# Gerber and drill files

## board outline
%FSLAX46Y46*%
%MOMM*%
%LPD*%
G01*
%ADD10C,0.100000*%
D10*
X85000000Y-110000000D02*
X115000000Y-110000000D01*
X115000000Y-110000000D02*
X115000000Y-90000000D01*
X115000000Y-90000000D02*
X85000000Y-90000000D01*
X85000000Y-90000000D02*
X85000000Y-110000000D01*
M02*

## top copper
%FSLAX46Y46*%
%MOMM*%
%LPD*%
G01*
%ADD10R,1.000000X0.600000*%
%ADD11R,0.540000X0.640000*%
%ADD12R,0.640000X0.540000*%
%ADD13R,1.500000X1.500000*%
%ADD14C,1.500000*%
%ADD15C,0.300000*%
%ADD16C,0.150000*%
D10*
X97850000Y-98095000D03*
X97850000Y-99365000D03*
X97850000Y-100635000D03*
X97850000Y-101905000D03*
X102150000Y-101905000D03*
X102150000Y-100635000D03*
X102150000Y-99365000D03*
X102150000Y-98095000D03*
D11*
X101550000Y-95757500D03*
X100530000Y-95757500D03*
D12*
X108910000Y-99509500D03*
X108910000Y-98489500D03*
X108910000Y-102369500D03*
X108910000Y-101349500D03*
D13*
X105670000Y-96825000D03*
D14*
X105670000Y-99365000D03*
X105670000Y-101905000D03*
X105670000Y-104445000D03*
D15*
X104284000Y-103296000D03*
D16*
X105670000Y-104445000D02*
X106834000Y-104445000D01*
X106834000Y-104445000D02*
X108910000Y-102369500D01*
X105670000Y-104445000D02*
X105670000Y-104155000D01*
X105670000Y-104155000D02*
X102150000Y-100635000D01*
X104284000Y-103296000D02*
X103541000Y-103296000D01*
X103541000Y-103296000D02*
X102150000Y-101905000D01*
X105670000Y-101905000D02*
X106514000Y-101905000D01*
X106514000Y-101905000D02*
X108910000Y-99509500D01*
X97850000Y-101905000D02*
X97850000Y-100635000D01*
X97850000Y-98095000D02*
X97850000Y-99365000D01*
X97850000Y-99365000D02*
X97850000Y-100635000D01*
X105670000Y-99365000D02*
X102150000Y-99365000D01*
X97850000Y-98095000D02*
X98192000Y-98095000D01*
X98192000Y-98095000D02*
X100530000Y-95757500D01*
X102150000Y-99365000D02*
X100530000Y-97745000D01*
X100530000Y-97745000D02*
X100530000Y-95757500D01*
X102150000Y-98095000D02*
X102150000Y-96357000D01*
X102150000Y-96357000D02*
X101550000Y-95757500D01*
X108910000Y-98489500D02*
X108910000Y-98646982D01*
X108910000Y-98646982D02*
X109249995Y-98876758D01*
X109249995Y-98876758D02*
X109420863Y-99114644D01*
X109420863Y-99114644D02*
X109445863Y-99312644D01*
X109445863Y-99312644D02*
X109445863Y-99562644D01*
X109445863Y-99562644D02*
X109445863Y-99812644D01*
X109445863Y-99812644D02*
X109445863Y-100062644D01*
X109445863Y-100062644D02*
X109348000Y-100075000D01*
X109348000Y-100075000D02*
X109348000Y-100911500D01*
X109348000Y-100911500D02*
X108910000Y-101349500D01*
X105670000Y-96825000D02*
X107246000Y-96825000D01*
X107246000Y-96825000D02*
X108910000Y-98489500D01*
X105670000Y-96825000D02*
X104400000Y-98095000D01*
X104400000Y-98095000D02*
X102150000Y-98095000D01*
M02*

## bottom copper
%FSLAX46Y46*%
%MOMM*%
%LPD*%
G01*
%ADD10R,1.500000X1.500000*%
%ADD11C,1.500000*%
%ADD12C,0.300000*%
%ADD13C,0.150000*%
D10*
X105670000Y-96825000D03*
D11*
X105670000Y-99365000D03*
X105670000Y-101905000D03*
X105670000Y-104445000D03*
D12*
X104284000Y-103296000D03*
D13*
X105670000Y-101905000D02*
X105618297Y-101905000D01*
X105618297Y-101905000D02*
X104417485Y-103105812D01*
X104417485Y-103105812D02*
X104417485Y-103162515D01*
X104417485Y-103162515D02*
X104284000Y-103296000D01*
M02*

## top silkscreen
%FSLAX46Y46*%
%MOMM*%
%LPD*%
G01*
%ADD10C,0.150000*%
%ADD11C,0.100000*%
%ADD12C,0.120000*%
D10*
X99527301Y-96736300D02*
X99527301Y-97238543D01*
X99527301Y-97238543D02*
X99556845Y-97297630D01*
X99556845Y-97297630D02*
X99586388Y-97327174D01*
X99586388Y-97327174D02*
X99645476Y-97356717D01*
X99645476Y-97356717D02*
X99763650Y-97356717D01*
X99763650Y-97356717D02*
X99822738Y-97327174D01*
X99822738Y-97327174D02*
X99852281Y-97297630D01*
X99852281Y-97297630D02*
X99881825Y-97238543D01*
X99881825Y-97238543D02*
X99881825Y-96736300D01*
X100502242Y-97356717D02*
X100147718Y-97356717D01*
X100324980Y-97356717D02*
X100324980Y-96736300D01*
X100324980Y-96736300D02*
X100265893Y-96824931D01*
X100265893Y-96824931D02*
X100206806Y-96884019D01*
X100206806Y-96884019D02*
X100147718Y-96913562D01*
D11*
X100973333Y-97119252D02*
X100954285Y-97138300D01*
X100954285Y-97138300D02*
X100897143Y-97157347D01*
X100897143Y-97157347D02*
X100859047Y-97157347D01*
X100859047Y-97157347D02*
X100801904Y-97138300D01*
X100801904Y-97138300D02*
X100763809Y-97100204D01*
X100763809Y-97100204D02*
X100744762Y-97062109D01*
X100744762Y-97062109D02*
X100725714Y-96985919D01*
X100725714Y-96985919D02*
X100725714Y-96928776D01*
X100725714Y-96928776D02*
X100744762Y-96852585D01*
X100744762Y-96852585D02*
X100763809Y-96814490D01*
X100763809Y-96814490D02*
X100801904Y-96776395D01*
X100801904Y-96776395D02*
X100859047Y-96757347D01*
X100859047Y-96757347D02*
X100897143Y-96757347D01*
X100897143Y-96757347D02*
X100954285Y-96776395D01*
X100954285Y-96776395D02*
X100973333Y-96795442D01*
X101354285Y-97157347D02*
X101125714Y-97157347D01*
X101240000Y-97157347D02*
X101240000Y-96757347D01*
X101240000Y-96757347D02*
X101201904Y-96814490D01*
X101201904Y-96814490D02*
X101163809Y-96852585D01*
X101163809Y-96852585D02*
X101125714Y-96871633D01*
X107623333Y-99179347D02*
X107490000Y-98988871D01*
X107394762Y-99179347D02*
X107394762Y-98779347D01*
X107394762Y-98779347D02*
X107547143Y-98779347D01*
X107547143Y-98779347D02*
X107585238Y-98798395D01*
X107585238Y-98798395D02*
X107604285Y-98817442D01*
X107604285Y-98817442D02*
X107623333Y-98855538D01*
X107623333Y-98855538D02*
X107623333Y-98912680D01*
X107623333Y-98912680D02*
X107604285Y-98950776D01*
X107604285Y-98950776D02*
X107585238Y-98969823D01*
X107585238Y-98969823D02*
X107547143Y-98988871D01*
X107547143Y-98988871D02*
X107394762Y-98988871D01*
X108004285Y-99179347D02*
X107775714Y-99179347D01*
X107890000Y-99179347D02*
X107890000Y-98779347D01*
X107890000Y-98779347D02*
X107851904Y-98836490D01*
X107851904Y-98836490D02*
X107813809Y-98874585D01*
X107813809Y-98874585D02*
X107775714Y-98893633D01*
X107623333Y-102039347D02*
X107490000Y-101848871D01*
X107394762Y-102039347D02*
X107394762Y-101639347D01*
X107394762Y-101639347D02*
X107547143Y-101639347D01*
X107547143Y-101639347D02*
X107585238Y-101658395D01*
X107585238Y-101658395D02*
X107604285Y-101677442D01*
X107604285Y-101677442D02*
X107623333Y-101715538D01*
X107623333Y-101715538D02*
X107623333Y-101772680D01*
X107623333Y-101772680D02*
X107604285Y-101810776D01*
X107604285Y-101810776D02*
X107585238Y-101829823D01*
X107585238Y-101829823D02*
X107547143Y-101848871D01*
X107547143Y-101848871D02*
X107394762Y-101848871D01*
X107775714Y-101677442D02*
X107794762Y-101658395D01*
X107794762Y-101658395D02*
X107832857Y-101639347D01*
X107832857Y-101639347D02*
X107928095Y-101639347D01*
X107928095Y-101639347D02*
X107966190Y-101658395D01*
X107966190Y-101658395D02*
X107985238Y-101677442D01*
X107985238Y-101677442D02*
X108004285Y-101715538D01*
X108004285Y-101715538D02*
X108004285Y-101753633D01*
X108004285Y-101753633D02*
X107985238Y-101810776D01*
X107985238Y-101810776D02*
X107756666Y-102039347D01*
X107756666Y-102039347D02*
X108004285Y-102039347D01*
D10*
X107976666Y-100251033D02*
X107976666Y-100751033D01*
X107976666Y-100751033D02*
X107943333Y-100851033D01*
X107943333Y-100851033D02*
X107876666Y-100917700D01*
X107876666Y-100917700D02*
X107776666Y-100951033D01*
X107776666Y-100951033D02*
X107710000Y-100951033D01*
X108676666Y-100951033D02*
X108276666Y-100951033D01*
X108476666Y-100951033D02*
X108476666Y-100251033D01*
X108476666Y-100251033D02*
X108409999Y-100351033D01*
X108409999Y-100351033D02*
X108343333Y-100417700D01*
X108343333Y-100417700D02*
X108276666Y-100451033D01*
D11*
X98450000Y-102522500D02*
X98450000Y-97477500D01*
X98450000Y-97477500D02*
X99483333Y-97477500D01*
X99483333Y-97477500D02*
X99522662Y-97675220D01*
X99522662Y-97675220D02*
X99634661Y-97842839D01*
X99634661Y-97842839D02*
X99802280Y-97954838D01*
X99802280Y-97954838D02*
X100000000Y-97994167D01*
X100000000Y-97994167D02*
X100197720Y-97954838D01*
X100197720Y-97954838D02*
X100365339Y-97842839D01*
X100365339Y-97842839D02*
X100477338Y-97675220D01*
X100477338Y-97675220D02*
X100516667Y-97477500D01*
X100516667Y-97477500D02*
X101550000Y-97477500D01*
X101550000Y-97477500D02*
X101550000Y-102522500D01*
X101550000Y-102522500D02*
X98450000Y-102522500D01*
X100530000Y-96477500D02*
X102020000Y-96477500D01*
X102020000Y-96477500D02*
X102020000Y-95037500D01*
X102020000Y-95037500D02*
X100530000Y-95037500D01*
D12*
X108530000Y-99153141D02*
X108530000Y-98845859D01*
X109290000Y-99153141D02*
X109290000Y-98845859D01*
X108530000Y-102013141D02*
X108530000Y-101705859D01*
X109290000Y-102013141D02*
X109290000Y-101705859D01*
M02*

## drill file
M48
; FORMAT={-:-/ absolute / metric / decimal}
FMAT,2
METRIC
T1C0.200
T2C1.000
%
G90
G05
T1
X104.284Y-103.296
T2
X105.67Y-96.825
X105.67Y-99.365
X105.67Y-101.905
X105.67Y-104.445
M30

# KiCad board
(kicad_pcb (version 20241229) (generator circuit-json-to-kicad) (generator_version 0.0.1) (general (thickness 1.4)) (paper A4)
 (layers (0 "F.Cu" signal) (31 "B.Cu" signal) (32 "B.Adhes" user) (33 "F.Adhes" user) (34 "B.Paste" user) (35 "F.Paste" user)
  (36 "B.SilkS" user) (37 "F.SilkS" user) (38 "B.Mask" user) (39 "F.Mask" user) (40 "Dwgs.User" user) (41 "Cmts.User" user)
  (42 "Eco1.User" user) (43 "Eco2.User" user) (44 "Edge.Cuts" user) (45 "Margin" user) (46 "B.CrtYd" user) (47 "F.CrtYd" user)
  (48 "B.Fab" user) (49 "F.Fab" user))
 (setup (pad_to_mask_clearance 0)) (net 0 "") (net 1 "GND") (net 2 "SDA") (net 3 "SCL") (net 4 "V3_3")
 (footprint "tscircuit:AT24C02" (layer F.Cu) (at 100 100 0)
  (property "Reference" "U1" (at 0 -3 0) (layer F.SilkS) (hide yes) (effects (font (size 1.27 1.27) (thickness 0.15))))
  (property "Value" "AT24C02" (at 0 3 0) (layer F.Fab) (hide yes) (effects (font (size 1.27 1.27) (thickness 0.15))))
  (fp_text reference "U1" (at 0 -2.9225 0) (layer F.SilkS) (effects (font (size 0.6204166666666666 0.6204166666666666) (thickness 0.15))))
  (fp_line (start -1.5499999999999998 2.5225) (end -1.5499999999999998 -2.5225) (stroke (width 0.1) (type default)) (layer F.SilkS))
  (fp_line (start -1.5499999999999998 -2.5225) (end -0.5166666666666666 -2.5225) (stroke (width 0.1) (type default)) (layer F.SilkS))
  (fp_line (start -0.5166666666666666 -2.5225) (end -0.47733775846416476 -2.32478022661137) (stroke (width 0.1) (type default))
   (layer F.SilkS))
  (fp_line (start -0.47733775846416476 -2.32478022661137) (end -0.3653385036130495 -2.1571614963869505) (stroke (width 0.1) (type default))
   (layer F.SilkS))
  (fp_line (start -0.3653385036130495 -2.1571614963869505) (end -0.19771977338862967 -2.0451622415358353)
   (stroke (width 0.1) (type default)) (layer F.SilkS))
  (fp_line (start -0.19771977338862967 -2.0451622415358353) (end 3.1636708977973285e-17 -2.0058333333333334)
   (stroke (width 0.1) (type default)) (layer F.SilkS))
  (fp_line (start 3.1636708977973285e-17 -2.0058333333333334) (end 0.1977197733886297 -2.0451622415358353)
   (stroke (width 0.1) (type default)) (layer F.SilkS))
  (fp_line (start 0.1977197733886297 -2.0451622415358353) (end 0.3653385036130496 -2.1571614963869505) (stroke (width 0.1) (type default))
   (layer F.SilkS))
  (fp_line (start 0.3653385036130496 -2.1571614963869505) (end 0.47733775846416476 -2.32478022661137) (stroke (width 0.1) (type default))
   (layer F.SilkS))
  (fp_line (start 0.47733775846416476 -2.32478022661137) (end 0.5166666666666666 -2.5225) (stroke (width 0.1) (type default))
   (layer F.SilkS))
  (fp_line (start 0.5166666666666666 -2.5225) (end 1.5499999999999998 -2.5225) (stroke (width 0.1) (type default)) (layer F.SilkS))
  (fp_line (start 1.5499999999999998 -2.5225) (end 1.5499999999999998 2.5225) (stroke (width 0.1) (type default)) (layer F.SilkS))
  (fp_line (start 1.5499999999999998 2.5225) (end -1.5499999999999998 2.5225) (stroke (width 0.1) (type default)) (layer F.SilkS))
  (pad "1" smd rect (at -2.15 -1.905 0) (size 1 0.6) (layers F.Cu F.Paste F.Mask) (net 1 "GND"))
  (pad "2" smd rect (at -2.15 -0.635 0) (size 1 0.6) (layers F.Cu F.Paste F.Mask) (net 1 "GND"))
  (pad "3" smd rect (at -2.15 0.635 0) (size 1 0.6) (layers F.Cu F.Paste F.Mask) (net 1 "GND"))
  (pad "4" smd rect (at -2.15 1.905 0) (size 1 0.6) (layers F.Cu F.Paste F.Mask) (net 1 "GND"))
  (pad "5" smd rect (at 2.15 1.905 0) (size 1 0.6) (layers F.Cu F.Paste F.Mask) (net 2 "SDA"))
  (pad "6" smd rect (at 2.15 0.635 0) (size 1 0.6) (layers F.Cu F.Paste F.Mask) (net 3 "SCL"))
  (pad "7" smd rect (at 2.15 -0.635 0) (size 1 0.6) (layers F.Cu F.Paste F.Mask) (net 1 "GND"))
  (pad "8" smd rect (at 2.15 -1.905 0) (size 1 0.6) (layers F.Cu F.Paste F.Mask) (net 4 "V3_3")))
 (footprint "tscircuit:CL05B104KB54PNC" (layer F.Cu) (at 101.04 95.7575 180)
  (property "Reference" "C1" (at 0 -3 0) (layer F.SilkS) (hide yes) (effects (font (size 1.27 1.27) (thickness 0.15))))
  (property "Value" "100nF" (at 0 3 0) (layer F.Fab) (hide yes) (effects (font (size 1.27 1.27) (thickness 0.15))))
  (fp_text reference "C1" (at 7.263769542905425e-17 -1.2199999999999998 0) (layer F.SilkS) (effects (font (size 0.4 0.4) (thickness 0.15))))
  (fp_line (start 0.51 -0.7199999999999999) (end -0.9800000000000001 -0.7200000000000001) (stroke (width 0.1) (type default))
   (layer F.SilkS))
  (fp_line (start -0.9800000000000001 -0.7200000000000001) (end -0.9799999999999999 0.7199999999999999) (stroke (width 0.1) (type default))
   (layer F.SilkS))
  (fp_line (start -0.9799999999999999 0.7199999999999999) (end 0.51 0.7199999999999996) (stroke (width 0.1) (type default)) (layer F.SilkS))
  (pad "1" smd rect (at -0.51 0 0) (size 0.54 0.64) (layers F.Cu F.Paste F.Mask) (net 4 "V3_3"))
  (pad "2" smd rect (at 0.5100000000000001 0 0) (size 0.54 0.64) (layers F.Cu F.Paste F.Mask) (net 1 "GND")))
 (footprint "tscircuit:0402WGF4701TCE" (layer F.Cu) (at 108.91 98.9995 90)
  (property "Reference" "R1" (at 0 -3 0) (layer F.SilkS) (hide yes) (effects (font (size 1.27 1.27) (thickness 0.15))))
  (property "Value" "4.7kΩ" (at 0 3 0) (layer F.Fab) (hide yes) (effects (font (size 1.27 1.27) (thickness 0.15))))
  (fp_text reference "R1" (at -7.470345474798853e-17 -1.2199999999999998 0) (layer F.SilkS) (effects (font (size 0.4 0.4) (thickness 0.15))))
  (fp_line (start -0.15364099999999994 -0.3800000000000008) (end 0.1536409999999999 -0.3800000000000008)
   (stroke (width 0.12) (type default)) (layer F.SilkS))
  (fp_line (start -0.153641 0.3800000000000008) (end 0.15364099999999994 0.3800000000000008) (stroke (width 0.12) (type default))
   (layer F.SilkS))
  (pad "1" smd rect (at -0.5099999999999999 0 0) (size 0.64 0.54) (layers F.Cu F.Paste F.Mask) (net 2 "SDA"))
  (pad "2" smd rect (at 0.51 0 0) (size 0.64 0.54) (layers F.Cu F.Paste F.Mask) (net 4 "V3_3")))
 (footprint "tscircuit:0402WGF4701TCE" (layer F.Cu) (at 108.91 101.8595 90)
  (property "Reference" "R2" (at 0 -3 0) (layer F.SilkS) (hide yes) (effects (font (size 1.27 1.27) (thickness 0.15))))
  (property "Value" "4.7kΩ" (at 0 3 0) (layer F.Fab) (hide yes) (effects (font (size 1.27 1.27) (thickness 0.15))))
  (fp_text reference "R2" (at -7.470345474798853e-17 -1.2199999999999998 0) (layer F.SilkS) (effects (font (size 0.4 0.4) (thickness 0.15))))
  (fp_line (start -0.15364099999999994 -0.3800000000000008) (end 0.1536409999999999 -0.3800000000000008)
   (stroke (width 0.12) (type default)) (layer F.SilkS))
  (fp_line (start -0.1536409999999999 0.3800000000000008) (end 0.15364099999999994 0.3800000000000008) (stroke (width 0.12) (type default))
   (layer F.SilkS))
  (pad "1" smd rect (at -0.5099999999999998 0 0) (size 0.64 0.54) (layers F.Cu F.Paste F.Mask) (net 3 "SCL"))
  (pad "2" smd rect (at 0.51 0 0) (size 0.64 0.54) (layers F.Cu F.Paste F.Mask) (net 4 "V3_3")))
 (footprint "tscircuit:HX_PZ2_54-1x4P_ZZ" (layer F.Cu) (at 105.67 100.635 -90.00000000000001)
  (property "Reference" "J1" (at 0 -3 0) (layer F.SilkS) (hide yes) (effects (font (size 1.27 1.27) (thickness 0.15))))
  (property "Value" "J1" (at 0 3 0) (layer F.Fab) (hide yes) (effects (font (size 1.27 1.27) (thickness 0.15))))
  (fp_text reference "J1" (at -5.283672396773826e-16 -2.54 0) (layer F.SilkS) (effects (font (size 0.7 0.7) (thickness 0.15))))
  (pad "1" thru_hole rect (at -3.81 5.705062545910424e-16 0) (size 1.5 1.5) (drill 1) (layers *.Cu *.Mask) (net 4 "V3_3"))
  (pad "2" thru_hole circle (at -1.27 4.862282247637226e-16 0) (size 1.5 1.5) (drill 1) (layers *.Cu *.Mask) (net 1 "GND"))
  (pad "3" thru_hole circle (at 1.27 -4.862282247637226e-16 0) (size 1.5 1.5) (drill 1) (layers *.Cu *.Mask) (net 2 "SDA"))
  (pad "4" thru_hole circle (at 3.8100000000000005 -5.705062545910426e-16 0) (size 1.5 1.5) (drill 1) (layers *.Cu *.Mask) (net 3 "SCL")))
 (segment (start 105.67 104.44500000000001) (end 106.834 104.44500000000001) (width 0.15) (layer F.Cu) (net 3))
 (segment (start 106.834 104.44500000000001) (end 108.91 102.3695) (width 0.15) (layer F.Cu) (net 3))
 (segment (start 105.67 104.44500000000001) (end 105.67 104.155) (width 0.15) (layer F.Cu) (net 3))
 (segment (start 105.67 104.155) (end 102.15 100.635) (width 0.15) (layer F.Cu) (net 3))
 (segment (start 105.67 101.905) (end 105.61829742994085 101.905) (width 0.15) (layer B.Cu) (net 2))
 (segment (start 105.61829742994085 101.905) (end 104.41748540321385 103.10581202672702) (width 0.15) (layer B.Cu) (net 2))
 (segment (start 104.41748540321385 103.10581202672702) (end 104.41748540321385 103.16251459678615) (width 0.15) (layer B.Cu) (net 2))
 (segment (start 104.41748540321385 103.16251459678615) (end 104.284 103.296) (width 0.15) (layer B.Cu) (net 2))
 (segment (start 104.284 103.296) (end 103.541 103.296) (width 0.15) (layer F.Cu) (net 2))
 (segment (start 103.541 103.296) (end 102.15 101.905) (width 0.15) (layer F.Cu) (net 2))
 (segment (start 105.67 101.905) (end 106.514 101.905) (width 0.15) (layer F.Cu) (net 2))
 (segment (start 106.514 101.905) (end 108.91 99.5095) (width 0.15) (layer F.Cu) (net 2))
 (segment (start 97.85 101.905) (end 97.85 100.635) (width 0.15) (layer F.Cu) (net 1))
 (segment (start 97.85 98.095) (end 97.85 99.365) (width 0.15) (layer F.Cu) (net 1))
 (segment (start 97.85 99.365) (end 97.85 100.635) (width 0.15) (layer F.Cu) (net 1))
 (segment (start 105.67 99.365) (end 102.15 99.365) (width 0.15) (layer F.Cu) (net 1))
 (segment (start 97.85 98.095) (end 98.192 98.095) (width 0.15) (layer F.Cu) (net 1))
 (segment (start 98.192 98.095) (end 100.53 95.7575) (width 0.15) (layer F.Cu) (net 1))
 (segment (start 102.15 99.365) (end 100.53 97.745) (width 0.15) (layer F.Cu) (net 1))
 (segment (start 100.53 97.745) (end 100.53 95.7575) (width 0.15) (layer F.Cu) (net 1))
 (segment (start 102.15 98.095) (end 102.15 96.357) (width 0.15) (layer F.Cu) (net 4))
 (segment (start 102.15 96.357) (end 101.55 95.7575) (width 0.15) (layer F.Cu) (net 4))
 (segment (start 108.91 98.48949999999999) (end 108.91 98.64698194937783) (width 0.15) (layer F.Cu) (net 4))
 (segment (start 108.91 98.64698194937783) (end 109.24999537270699 98.87675797422321) (width 0.15) (layer F.Cu) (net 4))
 (segment (start 109.24999537270699 98.87675797422321) (end 109.42086291872914 99.11464357086753) (width 0.15) (layer F.Cu) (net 4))
 (segment (start 109.42086291872914 99.11464357086753) (end 109.44586291872915 99.31264357086754) (width 0.15) (layer F.Cu) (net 4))
 (segment (start 109.44586291872915 99.31264357086754) (end 109.44586291872915 99.56264357086754) (width 0.15) (layer F.Cu) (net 4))
 (segment (start 109.44586291872915 99.56264357086754) (end 109.44586291872915 99.81264357086754) (width 0.15) (layer F.Cu) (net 4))
 (segment (start 109.44586291872915 99.81264357086754) (end 109.44586291872915 100.06264357086754) (width 0.15) (layer F.Cu) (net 4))
 (segment (start 109.44586291872915 100.06264357086754) (end 109.348 100.075) (width 0.15) (layer F.Cu) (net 4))
 (segment (start 109.348 100.075) (end 109.348 100.9115) (width 0.15) (layer F.Cu) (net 4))
 (segment (start 109.348 100.9115) (end 108.91 101.3495) (width 0.15) (layer F.Cu) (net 4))
 (segment (start 105.67 96.825) (end 107.246 96.825) (width 0.15) (layer F.Cu) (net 4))
 (segment (start 107.246 96.825) (end 108.91 98.48949999999999) (width 0.15) (layer F.Cu) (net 4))
 (segment (start 105.67 96.825) (end 104.4 98.095) (width 0.15) (layer F.Cu) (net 4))
 (segment (start 104.4 98.095) (end 102.15 98.095) (width 0.15) (layer F.Cu) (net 4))
 (gr_line (start 85 110) (end 115 110) (width 0.1) (layer Edge.Cuts))
 (gr_line (start 115 110) (end 115 90) (width 0.1) (layer Edge.Cuts))
 (gr_line (start 115 90) (end 85 90) (width 0.1) (layer Edge.Cuts))
 (gr_line (start 85 90) (end 85 110) (width 0.1) (layer Edge.Cuts))
 (via (at 104.284 103.296) (size 0.3) (drill 0.2) (layers F.Cu B.Cu) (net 2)))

